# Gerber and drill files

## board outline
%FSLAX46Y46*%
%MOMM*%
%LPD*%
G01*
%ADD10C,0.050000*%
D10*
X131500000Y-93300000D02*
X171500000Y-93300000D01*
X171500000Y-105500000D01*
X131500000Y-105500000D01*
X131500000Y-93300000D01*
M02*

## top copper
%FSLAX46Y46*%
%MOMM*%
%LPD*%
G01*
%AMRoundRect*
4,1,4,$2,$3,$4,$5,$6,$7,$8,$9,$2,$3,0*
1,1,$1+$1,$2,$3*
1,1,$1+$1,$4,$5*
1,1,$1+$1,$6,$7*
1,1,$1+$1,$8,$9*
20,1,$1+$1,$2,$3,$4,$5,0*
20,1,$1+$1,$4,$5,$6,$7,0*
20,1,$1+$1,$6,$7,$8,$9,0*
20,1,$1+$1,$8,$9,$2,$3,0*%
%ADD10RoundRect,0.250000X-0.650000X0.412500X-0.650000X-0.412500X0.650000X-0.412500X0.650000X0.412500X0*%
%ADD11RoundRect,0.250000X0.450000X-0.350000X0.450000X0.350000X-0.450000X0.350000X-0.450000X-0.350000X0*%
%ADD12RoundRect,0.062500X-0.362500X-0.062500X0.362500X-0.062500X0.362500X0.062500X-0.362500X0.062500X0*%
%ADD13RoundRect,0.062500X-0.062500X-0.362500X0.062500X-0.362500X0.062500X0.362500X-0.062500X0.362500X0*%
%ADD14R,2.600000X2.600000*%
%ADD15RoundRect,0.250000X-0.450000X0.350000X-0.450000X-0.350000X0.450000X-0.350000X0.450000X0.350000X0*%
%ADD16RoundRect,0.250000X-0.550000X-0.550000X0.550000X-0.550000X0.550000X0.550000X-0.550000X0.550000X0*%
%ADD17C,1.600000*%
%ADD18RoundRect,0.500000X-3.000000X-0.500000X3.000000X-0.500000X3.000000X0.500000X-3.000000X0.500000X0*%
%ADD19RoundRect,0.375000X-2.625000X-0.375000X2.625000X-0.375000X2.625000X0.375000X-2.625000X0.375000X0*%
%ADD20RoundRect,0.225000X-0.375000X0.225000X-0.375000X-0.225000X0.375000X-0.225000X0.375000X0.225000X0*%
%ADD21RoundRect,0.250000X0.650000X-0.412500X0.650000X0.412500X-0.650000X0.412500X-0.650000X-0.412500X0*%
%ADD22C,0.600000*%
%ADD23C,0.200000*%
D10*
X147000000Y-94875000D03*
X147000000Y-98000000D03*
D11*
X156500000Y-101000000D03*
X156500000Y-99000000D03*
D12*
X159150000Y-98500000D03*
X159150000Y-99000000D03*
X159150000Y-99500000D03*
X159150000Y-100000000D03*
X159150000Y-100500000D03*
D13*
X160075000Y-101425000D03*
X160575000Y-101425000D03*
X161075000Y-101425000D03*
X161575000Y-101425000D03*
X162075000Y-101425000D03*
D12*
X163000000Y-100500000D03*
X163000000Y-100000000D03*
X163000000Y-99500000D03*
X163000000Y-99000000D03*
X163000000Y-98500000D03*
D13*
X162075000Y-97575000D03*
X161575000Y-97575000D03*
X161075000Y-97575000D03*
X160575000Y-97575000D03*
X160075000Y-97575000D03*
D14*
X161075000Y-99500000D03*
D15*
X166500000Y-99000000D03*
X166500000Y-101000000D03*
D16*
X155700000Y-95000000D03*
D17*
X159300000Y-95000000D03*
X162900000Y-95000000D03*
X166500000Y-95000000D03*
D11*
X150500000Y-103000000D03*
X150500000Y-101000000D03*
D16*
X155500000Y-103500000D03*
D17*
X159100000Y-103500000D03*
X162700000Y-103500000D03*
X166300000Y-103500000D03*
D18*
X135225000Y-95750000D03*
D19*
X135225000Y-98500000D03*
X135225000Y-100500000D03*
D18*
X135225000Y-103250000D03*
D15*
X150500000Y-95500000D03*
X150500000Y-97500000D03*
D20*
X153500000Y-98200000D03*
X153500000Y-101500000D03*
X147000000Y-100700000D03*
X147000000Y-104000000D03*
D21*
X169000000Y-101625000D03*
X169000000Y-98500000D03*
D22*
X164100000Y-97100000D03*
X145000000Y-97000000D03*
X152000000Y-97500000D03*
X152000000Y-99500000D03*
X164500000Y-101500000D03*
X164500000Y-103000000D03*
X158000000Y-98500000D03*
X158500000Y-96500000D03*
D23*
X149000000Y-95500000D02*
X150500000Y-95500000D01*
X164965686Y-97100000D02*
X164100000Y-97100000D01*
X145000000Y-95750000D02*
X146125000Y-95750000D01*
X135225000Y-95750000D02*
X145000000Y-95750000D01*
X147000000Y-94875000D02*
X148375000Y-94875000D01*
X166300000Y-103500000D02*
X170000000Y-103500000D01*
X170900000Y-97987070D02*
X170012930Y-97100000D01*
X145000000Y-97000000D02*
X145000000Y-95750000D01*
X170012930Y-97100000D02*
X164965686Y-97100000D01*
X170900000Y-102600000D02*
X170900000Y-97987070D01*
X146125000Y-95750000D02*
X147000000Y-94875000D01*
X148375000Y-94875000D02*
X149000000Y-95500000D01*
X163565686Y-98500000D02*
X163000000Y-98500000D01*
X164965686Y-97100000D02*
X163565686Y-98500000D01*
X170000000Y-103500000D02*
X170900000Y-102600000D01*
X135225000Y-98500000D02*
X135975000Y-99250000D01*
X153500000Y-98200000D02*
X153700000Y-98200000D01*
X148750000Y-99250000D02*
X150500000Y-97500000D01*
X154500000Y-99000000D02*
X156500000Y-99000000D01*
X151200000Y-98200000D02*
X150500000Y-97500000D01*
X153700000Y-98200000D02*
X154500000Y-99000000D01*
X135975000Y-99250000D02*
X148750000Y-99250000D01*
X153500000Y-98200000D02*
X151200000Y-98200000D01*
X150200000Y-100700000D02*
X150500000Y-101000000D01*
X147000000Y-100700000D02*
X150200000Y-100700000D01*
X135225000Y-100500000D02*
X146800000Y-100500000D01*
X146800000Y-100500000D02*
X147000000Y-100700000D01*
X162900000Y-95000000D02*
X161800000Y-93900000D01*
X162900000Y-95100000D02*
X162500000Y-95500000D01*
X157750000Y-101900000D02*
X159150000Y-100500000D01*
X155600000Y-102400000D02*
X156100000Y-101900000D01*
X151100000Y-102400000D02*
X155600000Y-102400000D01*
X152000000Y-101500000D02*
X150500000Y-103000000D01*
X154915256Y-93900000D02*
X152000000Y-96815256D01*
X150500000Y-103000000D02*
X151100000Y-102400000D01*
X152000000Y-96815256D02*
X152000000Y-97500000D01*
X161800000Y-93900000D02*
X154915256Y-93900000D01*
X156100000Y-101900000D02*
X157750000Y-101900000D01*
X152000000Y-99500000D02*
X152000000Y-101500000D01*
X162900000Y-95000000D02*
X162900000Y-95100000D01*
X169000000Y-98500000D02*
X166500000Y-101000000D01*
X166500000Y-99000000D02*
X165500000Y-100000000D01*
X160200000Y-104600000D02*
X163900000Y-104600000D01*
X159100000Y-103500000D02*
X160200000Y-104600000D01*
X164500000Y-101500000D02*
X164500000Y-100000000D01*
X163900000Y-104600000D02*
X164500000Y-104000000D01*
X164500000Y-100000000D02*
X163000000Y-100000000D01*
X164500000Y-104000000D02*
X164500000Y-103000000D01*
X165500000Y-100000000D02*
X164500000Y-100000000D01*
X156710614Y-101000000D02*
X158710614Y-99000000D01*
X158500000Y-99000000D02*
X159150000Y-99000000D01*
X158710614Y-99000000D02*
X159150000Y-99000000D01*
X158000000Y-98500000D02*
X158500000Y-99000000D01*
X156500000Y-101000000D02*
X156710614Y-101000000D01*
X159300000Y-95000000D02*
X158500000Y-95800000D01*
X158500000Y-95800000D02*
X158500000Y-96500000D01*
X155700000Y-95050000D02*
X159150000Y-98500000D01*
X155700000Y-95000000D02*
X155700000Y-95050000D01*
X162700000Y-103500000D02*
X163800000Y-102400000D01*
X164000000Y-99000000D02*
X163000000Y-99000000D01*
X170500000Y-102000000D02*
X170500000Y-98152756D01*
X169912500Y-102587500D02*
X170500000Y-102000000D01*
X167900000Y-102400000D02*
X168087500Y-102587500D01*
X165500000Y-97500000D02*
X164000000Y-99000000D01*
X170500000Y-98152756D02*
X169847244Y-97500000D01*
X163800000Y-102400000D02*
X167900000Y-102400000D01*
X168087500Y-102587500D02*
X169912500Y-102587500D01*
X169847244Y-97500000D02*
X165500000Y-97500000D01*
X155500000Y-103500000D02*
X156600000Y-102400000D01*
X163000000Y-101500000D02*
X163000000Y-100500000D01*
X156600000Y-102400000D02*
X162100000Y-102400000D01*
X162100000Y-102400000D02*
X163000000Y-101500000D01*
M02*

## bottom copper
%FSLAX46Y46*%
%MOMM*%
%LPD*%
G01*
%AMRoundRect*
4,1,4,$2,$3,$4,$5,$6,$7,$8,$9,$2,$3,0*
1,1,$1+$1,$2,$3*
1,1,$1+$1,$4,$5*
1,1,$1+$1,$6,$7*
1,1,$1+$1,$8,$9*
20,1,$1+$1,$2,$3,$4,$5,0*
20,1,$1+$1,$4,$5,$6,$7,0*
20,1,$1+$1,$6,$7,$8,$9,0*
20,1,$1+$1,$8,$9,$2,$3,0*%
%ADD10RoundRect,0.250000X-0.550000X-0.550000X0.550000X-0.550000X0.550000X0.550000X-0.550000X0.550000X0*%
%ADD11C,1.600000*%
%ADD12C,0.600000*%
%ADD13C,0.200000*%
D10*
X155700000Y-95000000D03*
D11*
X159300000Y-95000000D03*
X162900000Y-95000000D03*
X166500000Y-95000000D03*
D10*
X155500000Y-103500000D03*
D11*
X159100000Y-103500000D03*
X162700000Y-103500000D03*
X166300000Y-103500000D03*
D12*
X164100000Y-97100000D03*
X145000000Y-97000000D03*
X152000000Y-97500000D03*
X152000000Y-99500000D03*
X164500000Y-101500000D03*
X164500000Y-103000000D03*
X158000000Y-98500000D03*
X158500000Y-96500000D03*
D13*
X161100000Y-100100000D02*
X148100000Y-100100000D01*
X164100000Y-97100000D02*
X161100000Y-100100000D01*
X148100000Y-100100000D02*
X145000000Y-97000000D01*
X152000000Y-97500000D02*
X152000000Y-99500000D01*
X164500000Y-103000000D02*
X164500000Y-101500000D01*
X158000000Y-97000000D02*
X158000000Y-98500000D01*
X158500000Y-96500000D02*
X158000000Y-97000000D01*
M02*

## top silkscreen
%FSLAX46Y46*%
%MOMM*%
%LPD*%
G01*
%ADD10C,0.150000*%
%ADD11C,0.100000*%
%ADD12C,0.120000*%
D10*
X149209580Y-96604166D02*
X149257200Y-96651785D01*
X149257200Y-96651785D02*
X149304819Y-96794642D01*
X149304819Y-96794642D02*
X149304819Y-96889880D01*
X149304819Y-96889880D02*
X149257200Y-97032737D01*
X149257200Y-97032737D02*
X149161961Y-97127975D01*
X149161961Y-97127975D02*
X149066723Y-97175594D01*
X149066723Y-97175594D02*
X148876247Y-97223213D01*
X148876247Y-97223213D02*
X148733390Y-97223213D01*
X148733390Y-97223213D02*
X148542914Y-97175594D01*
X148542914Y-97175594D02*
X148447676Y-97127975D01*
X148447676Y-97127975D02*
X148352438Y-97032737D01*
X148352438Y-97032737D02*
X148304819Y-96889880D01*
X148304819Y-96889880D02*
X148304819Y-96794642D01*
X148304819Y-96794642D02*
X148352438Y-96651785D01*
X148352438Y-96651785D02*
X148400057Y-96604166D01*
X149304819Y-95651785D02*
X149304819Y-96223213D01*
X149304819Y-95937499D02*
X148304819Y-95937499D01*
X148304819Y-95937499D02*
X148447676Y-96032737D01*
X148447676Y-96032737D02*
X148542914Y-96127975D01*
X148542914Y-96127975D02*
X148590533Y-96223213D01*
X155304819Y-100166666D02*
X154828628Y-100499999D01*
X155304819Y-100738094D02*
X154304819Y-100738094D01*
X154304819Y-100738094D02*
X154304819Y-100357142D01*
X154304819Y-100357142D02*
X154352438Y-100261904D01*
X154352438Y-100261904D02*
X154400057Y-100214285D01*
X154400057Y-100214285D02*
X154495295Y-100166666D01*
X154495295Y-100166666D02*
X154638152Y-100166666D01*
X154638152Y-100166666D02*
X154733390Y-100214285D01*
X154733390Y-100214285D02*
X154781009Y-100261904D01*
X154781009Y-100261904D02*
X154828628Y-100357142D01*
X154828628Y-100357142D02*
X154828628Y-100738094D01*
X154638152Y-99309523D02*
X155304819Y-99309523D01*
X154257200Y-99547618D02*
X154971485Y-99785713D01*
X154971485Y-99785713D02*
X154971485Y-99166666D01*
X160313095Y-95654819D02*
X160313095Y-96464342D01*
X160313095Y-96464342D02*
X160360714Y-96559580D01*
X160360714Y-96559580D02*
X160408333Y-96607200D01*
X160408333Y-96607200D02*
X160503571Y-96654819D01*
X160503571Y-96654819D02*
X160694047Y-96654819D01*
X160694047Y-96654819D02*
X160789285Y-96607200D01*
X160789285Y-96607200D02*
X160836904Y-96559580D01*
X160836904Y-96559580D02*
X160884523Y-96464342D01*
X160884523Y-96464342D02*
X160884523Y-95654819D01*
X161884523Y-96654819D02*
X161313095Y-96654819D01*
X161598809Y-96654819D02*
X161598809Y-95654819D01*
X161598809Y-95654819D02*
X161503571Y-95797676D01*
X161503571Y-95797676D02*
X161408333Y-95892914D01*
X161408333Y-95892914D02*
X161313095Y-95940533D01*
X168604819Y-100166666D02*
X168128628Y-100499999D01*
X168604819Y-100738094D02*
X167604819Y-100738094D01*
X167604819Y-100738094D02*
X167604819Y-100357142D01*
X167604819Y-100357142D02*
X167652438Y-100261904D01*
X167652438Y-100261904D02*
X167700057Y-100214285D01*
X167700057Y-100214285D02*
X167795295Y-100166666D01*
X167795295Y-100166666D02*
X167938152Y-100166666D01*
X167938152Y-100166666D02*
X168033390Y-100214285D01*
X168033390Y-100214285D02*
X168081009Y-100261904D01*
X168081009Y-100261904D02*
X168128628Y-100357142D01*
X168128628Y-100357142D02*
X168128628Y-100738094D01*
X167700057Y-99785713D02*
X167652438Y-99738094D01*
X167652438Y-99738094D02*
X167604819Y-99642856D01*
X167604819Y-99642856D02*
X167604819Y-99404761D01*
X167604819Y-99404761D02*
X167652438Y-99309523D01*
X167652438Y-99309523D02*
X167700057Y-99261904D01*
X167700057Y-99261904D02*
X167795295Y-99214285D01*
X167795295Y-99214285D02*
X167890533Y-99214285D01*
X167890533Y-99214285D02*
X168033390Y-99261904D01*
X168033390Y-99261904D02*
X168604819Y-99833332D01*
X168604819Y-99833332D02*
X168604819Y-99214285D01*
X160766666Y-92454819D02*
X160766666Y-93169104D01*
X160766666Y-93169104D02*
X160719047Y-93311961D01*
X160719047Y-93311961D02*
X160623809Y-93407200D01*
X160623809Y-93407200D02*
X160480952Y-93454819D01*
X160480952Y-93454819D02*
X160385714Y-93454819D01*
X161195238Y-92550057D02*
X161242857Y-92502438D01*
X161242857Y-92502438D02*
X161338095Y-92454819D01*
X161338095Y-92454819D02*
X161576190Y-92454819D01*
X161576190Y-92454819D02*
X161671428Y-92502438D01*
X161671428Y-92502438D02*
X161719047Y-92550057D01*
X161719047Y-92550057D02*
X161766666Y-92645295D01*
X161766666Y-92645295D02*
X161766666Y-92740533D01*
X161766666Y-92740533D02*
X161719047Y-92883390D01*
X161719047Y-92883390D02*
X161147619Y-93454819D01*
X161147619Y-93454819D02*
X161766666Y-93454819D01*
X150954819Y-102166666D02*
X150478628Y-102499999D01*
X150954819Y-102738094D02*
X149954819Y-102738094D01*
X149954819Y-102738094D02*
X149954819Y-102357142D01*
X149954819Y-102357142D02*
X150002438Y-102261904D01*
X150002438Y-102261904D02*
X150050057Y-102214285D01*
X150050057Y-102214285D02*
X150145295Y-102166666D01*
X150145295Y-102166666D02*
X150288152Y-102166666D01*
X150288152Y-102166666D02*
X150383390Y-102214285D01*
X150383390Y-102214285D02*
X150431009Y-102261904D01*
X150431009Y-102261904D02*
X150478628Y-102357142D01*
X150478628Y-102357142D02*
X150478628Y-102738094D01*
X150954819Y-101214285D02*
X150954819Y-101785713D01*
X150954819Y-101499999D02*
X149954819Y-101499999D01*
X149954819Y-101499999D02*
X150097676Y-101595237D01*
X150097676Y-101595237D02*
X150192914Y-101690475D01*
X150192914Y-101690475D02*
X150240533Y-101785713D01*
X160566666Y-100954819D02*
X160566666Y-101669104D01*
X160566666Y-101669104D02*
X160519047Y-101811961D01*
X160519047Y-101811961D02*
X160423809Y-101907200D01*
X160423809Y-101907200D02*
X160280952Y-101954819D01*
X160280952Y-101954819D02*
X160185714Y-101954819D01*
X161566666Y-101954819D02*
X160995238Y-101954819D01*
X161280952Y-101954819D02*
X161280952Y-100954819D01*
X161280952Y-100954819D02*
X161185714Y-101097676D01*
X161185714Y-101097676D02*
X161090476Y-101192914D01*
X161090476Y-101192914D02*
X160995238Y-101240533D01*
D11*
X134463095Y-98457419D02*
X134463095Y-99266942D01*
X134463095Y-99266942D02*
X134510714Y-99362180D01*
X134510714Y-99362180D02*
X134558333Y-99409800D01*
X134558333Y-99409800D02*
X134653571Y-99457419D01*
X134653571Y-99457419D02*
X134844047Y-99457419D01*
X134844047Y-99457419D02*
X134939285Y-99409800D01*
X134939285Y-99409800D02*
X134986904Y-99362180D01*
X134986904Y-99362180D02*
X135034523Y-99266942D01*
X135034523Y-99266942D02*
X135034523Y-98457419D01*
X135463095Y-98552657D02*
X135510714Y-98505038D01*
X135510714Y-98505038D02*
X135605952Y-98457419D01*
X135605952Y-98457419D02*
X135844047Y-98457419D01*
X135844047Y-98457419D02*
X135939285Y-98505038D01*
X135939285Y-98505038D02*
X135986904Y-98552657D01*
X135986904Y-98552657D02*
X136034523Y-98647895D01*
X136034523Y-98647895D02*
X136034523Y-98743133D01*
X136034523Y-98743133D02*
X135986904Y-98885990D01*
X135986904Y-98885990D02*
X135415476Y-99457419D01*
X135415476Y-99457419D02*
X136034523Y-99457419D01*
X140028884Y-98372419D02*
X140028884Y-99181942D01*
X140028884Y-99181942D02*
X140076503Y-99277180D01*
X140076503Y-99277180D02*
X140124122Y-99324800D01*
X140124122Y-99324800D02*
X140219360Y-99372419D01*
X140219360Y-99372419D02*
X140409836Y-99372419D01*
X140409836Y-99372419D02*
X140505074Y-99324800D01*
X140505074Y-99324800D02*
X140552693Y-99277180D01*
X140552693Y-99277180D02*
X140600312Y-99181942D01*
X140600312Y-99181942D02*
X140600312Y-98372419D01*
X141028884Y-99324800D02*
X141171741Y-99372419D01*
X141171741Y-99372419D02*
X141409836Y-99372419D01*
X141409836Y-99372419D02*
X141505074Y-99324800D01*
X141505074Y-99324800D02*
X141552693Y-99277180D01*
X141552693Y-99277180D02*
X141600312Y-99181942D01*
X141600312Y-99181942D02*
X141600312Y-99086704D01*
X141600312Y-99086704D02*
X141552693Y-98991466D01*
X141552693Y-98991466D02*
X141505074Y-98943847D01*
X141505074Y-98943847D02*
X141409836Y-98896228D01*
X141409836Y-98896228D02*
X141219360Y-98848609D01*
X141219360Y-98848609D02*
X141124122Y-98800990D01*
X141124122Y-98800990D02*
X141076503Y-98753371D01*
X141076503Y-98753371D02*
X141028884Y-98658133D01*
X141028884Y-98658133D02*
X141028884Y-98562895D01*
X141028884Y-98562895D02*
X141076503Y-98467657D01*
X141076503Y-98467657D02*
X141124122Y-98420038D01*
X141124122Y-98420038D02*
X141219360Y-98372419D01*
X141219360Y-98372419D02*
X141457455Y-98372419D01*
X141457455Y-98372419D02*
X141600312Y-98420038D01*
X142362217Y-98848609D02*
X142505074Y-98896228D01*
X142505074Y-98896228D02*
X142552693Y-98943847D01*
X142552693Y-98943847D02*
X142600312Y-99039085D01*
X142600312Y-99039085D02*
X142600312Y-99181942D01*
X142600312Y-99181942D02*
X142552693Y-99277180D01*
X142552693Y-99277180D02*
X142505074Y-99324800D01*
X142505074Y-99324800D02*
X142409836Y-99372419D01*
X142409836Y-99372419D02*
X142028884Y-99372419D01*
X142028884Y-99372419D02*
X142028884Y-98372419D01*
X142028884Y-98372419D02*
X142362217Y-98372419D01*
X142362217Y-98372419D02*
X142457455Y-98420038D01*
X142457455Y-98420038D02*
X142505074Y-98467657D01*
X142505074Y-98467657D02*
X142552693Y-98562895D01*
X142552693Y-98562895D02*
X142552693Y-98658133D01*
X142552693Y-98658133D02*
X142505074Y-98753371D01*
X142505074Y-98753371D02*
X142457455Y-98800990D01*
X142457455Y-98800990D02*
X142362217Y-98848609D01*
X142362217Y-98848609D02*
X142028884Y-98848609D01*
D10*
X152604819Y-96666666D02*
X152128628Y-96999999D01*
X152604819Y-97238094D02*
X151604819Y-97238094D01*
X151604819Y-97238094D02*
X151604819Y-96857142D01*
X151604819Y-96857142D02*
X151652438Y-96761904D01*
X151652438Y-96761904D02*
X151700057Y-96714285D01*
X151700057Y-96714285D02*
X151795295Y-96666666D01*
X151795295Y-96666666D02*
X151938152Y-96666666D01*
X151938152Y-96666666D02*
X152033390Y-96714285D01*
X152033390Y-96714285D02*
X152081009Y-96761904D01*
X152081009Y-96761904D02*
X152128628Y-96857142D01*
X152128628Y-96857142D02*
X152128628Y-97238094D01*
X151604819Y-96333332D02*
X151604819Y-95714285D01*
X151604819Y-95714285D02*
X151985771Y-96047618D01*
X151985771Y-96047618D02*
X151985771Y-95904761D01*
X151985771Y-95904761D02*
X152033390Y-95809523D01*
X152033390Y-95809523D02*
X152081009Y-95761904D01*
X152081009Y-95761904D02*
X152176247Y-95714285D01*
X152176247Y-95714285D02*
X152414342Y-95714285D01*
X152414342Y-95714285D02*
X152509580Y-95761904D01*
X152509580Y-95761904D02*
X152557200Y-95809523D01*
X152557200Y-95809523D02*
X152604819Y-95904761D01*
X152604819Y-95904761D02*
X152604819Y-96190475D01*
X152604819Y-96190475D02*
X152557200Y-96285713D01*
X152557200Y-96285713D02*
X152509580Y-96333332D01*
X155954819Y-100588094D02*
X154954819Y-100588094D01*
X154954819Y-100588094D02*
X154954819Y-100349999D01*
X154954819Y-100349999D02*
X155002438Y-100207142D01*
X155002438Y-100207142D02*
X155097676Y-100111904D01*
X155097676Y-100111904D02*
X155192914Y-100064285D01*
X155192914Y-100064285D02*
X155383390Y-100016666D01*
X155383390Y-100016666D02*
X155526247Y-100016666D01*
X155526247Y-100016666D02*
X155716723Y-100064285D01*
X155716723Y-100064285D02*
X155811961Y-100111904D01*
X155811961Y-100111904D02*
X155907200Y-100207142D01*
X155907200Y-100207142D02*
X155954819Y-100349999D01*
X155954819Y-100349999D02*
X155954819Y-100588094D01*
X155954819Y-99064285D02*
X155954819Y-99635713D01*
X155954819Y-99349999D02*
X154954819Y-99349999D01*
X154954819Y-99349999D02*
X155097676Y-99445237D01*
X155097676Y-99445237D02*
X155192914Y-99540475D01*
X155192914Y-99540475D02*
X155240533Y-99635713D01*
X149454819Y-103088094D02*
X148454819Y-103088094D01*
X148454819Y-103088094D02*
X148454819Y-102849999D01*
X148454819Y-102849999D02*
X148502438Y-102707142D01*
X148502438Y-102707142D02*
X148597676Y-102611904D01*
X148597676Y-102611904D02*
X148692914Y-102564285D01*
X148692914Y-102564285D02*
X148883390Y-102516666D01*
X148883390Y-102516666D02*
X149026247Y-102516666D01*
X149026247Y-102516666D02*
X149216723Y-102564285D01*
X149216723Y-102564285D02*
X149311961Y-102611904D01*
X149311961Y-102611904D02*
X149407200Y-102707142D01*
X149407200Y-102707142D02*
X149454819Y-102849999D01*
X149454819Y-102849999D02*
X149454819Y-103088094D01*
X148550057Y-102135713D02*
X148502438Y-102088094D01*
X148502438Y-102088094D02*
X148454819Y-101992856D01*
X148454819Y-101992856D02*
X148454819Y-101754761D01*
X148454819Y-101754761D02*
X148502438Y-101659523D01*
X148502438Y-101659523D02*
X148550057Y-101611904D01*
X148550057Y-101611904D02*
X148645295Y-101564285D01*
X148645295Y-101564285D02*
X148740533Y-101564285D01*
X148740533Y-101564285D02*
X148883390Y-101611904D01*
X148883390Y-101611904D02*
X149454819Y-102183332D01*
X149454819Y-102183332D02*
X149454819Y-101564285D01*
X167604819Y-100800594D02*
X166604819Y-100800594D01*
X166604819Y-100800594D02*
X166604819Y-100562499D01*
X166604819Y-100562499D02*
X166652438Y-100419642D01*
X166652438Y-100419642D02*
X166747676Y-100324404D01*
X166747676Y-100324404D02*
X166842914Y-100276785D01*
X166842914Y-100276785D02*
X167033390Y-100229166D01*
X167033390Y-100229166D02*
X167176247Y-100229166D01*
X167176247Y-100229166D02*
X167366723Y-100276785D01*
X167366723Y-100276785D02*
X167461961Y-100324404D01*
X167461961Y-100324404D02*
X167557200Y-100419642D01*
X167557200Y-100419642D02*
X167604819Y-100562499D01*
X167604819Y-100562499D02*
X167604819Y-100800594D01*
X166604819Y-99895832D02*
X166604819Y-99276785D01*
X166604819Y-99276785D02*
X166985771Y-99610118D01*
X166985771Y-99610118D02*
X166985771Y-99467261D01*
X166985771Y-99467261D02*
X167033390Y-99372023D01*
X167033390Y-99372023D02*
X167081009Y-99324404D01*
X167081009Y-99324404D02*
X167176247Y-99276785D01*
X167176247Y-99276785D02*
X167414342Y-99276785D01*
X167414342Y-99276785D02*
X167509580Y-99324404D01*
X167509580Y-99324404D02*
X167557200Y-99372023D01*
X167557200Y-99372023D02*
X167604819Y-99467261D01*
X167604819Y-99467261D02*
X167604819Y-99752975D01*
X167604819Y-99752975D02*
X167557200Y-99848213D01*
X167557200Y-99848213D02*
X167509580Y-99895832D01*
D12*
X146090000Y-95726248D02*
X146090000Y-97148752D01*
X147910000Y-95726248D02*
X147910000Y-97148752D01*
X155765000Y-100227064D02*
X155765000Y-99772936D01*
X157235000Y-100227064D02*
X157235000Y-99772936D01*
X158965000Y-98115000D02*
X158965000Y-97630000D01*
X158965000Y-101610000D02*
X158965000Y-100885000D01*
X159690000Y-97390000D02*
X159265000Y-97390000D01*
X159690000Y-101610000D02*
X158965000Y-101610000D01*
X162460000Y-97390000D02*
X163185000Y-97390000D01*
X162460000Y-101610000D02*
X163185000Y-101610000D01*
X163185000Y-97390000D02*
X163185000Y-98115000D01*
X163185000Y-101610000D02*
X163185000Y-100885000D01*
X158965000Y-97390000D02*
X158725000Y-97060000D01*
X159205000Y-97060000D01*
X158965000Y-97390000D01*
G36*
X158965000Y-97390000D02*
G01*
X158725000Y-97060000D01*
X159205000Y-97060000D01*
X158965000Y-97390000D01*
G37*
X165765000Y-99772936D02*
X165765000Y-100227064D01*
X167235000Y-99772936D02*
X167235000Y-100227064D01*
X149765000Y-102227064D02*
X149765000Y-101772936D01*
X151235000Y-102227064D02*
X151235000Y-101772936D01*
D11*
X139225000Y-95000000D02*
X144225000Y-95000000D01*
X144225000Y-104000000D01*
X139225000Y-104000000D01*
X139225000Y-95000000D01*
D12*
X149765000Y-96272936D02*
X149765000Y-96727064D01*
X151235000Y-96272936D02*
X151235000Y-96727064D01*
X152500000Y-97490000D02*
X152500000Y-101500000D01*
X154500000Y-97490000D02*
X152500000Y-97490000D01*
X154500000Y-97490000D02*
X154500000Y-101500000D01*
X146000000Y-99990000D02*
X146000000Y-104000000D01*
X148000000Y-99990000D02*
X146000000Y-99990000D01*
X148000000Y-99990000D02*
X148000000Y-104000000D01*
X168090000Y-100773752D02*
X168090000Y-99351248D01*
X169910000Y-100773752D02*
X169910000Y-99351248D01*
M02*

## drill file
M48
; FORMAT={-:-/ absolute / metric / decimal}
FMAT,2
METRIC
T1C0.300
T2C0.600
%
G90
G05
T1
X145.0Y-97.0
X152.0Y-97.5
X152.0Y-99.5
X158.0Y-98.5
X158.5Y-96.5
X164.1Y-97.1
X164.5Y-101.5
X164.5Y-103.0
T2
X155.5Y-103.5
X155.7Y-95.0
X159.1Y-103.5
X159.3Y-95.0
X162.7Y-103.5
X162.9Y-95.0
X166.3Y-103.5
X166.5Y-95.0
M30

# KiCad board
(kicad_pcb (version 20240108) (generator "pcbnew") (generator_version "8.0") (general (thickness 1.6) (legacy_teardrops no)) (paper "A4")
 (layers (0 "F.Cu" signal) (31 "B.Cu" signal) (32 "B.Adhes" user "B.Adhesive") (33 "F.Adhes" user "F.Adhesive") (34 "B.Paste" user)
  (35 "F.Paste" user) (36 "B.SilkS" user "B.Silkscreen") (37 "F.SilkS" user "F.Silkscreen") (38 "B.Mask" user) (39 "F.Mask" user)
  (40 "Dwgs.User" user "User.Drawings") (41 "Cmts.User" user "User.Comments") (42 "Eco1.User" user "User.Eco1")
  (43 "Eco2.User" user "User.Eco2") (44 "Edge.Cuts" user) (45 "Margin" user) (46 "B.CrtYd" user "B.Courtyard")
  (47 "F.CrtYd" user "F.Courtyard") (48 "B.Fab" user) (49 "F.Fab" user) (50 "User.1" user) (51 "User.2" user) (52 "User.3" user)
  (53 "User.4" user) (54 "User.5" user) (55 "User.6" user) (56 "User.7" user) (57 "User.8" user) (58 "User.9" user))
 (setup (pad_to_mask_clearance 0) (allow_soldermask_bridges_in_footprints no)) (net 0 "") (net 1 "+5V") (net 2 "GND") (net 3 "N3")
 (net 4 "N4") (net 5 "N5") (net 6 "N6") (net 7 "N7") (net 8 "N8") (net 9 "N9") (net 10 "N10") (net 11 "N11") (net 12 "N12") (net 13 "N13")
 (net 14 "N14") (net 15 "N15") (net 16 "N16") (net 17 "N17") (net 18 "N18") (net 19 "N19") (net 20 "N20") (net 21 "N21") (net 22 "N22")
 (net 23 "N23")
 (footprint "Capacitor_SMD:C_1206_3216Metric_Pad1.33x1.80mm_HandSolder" (layer "F.Cu") (at 147 96.4375 -90)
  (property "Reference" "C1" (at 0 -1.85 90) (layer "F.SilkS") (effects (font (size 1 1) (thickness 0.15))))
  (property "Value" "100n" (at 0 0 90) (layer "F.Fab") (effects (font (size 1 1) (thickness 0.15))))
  (fp_line (start -0.711252 0.91) (end 0.711252 0.91) (stroke (width 0.12) (type solid)) (layer "F.SilkS"))
  (fp_line (start -0.711252 -0.91) (end 0.711252 -0.91) (stroke (width 0.12) (type solid)) (layer "F.SilkS"))
  (pad "1" smd roundrect (at -1.5625 0 270) (size 1.325 1.8) (layers "F.Cu" "F.Paste" "F.Mask") (roundrect_rratio 0.188679) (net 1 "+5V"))
  (pad "2" smd roundrect (at 1.5625 0 270) (size 1.325 1.8) (layers "F.Cu" "F.Paste" "F.Mask") (roundrect_rratio 0.188679) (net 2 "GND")))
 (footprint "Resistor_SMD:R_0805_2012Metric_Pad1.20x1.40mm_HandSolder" (layer "F.Cu") (at 156.5 100 90)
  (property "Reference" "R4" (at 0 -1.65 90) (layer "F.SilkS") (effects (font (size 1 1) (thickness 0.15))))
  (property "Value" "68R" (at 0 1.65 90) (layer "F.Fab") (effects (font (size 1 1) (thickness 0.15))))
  (fp_line (start -0.227064 -0.735) (end 0.227064 -0.735) (stroke (width 0.12) (type solid)) (layer "F.SilkS"))
  (fp_line (start -0.227064 0.735) (end 0.227064 0.735) (stroke (width 0.12) (type solid)) (layer "F.SilkS"))
  (pad "1" smd roundrect (at -1 0 90) (size 1.2 1.4) (layers "F.Cu" "F.Paste" "F.Mask") (roundrect_rratio 0.208333) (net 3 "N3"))
  (pad "2" smd roundrect (at 1 0 90) (size 1.2 1.4) (layers "F.Cu" "F.Paste" "F.Mask") (roundrect_rratio 0.208333) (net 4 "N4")))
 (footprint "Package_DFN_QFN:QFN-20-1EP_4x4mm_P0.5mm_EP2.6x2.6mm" (layer "F.Cu") (at 161.075 99.5)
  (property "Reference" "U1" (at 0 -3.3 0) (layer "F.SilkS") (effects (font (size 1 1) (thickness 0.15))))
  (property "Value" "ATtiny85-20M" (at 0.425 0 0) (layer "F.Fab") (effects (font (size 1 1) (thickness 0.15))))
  (fp_line (start -2.11 -1.385) (end -2.11 -1.87) (stroke (width 0.12) (type solid)) (layer "F.SilkS"))
  (fp_line (start -2.11 2.11) (end -2.11 1.385) (stroke (width 0.12) (type solid)) (layer "F.SilkS"))
  (fp_line (start -1.385 -2.11) (end -1.81 -2.11) (stroke (width 0.12) (type solid)) (layer "F.SilkS"))
  (fp_line (start -1.385 2.11) (end -2.11 2.11) (stroke (width 0.12) (type solid)) (layer "F.SilkS"))
  (fp_line (start 1.385 -2.11) (end 2.11 -2.11) (stroke (width 0.12) (type solid)) (layer "F.SilkS"))
  (fp_line (start 1.385 2.11) (end 2.11 2.11) (stroke (width 0.12) (type solid)) (layer "F.SilkS"))
  (fp_line (start 2.11 -2.11) (end 2.11 -1.385) (stroke (width 0.12) (type solid)) (layer "F.SilkS"))
  (fp_line (start 2.11 2.11) (end 2.11 1.385) (stroke (width 0.12) (type solid)) (layer "F.SilkS"))
  (fp_poly
   (pts (xy -2.11 -2.11) (xy -2.35 -2.44) (xy -1.87 -2.44) (xy -2.11 -2.11)) (stroke (width 0.12) (type solid)) (fill solid)
   (layer "F.SilkS"))
  (pad "" smd roundrect (at -0.65 -0.65) (size 1.05 1.05) (layers "F.Paste") (roundrect_rratio 0.238095))
  (pad "" smd roundrect (at -0.65 0.65) (size 1.05 1.05) (layers "F.Paste") (roundrect_rratio 0.238095))
  (pad "" smd roundrect (at 0.65 -0.65) (size 1.05 1.05) (layers "F.Paste") (roundrect_rratio 0.238095))
  (pad "" smd roundrect (at 0.65 0.65) (size 1.05 1.05) (layers "F.Paste") (roundrect_rratio 0.238095))
  (pad "1" smd roundrect (at -1.925 -1) (size 0.85 0.25) (layers "F.Cu" "F.Paste" "F.Mask") (roundrect_rratio 0.25) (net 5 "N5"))
  (pad "2" smd roundrect (at -1.925 -0.5) (size 0.85 0.25) (layers "F.Cu" "F.Paste" "F.Mask") (roundrect_rratio 0.25) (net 3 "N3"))
  (pad "3" smd roundrect (at -1.925 0) (size 0.85 0.25) (layers "F.Cu" "F.Paste" "F.Mask") (roundrect_rratio 0.25) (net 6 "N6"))
  (pad "4" smd roundrect (at -1.925 0.5) (size 0.85 0.25) (layers "F.Cu" "F.Paste" "F.Mask") (roundrect_rratio 0.25) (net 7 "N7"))
  (pad "5" smd roundrect (at -1.925 1) (size 0.85 0.25) (layers "F.Cu" "F.Paste" "F.Mask") (roundrect_rratio 0.25) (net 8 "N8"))
  (pad "6" smd roundrect (at -1 1.925) (size 0.25 0.85) (layers "F.Cu" "F.Paste" "F.Mask") (roundrect_rratio 0.25) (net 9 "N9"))
  (pad "7" smd roundrect (at -0.5 1.925) (size 0.25 0.85) (layers "F.Cu" "F.Paste" "F.Mask") (roundrect_rratio 0.25) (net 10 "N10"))
  (pad "8" smd roundrect (at 0 1.925) (size 0.25 0.85) (layers "F.Cu" "F.Paste" "F.Mask") (roundrect_rratio 0.25) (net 2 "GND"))
  (pad "9" smd roundrect (at 0.5 1.925) (size 0.25 0.85) (layers "F.Cu" "F.Paste" "F.Mask") (roundrect_rratio 0.25) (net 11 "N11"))
  (pad "10" smd roundrect (at 1 1.925) (size 0.25 0.85) (layers "F.Cu" "F.Paste" "F.Mask") (roundrect_rratio 0.25) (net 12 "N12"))
  (pad "11" smd roundrect (at 1.925 1) (size 0.85 0.25) (layers "F.Cu" "F.Paste" "F.Mask") (roundrect_rratio 0.25) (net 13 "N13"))
  (pad "12" smd roundrect (at 1.925 0.5) (size 0.85 0.25) (layers "F.Cu" "F.Paste" "F.Mask") (roundrect_rratio 0.25) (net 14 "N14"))
  (pad "13" smd roundrect (at 1.925 0) (size 0.85 0.25) (layers "F.Cu" "F.Paste" "F.Mask") (roundrect_rratio 0.25) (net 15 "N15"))
  (pad "14" smd roundrect (at 1.925 -0.5) (size 0.85 0.25) (layers "F.Cu" "F.Paste" "F.Mask") (roundrect_rratio 0.25) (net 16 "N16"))
  (pad "15" smd roundrect (at 1.925 -1) (size 0.85 0.25) (layers "F.Cu" "F.Paste" "F.Mask") (roundrect_rratio 0.25) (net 1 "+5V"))
  (pad "16" smd roundrect (at 1 -1.925) (size 0.25 0.85) (layers "F.Cu" "F.Paste" "F.Mask") (roundrect_rratio 0.25) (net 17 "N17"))
  (pad "17" smd roundrect (at 0.5 -1.925) (size 0.25 0.85) (layers "F.Cu" "F.Paste" "F.Mask") (roundrect_rratio 0.25) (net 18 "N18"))
  (pad "18" smd roundrect (at 0 -1.925) (size 0.25 0.85) (layers "F.Cu" "F.Paste" "F.Mask") (roundrect_rratio 0.25) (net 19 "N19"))
  (pad "19" smd roundrect (at -0.5 -1.925) (size 0.25 0.85) (layers "F.Cu" "F.Paste" "F.Mask") (roundrect_rratio 0.25) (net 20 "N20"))
  (pad "20" smd roundrect (at -1 -1.925) (size 0.25 0.85) (layers "F.Cu" "F.Paste" "F.Mask") (roundrect_rratio 0.25) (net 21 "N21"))
  (pad "21" smd rect (at 0 0) (size 2.6 2.6) (layers "F.Cu" "F.Mask") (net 2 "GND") (zone_connect 2)))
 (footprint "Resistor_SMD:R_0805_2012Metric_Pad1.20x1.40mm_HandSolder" (layer "F.Cu") (at 166.5 100 -90)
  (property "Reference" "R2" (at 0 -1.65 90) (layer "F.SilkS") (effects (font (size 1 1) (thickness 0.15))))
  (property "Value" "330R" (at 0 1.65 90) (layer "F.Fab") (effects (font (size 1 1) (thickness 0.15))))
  (fp_line (start -0.227064 0.735) (end 0.227064 0.735) (stroke (width 0.12) (type solid)) (layer "F.SilkS"))
  (fp_line (start -0.227064 -0.735) (end 0.227064 -0.735) (stroke (width 0.12) (type solid)) (layer "F.SilkS"))
  (pad "1" smd roundrect (at -1 0 270) (size 1.2 1.4) (layers "F.Cu" "F.Paste" "F.Mask") (roundrect_rratio 0.208333) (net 14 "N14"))
  (pad "2" smd roundrect (at 1 0 270) (size 1.2 1.4) (layers "F.Cu" "F.Paste" "F.Mask") (roundrect_rratio 0.208333) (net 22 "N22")))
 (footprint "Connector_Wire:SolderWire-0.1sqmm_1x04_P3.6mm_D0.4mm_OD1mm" (layer "F.Cu") (at 155.7 95)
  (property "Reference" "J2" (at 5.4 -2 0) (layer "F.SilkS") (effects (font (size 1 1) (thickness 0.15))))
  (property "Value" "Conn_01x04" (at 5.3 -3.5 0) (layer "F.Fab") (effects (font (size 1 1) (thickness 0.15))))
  (pad "1" thru_hole roundrect (at 0 0) (size 1.6 1.6) (drill 0.6) (layers "*.Cu" "*.Mask") (remove_unused_layers no)
   (roundrect_rratio 0.15625) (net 5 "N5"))
  (pad "2" thru_hole circle (at 3.6 0) (size 1.6 1.6) (drill 0.6) (layers "*.Cu" "*.Mask") (remove_unused_layers no) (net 3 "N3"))
  (pad "3" thru_hole circle (at 7.2 0) (size 1.6 1.6) (drill 0.6) (layers "*.Cu" "*.Mask") (remove_unused_layers no) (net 8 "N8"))
  (pad "4" thru_hole circle (at 10.8 0) (size 1.6 1.6) (drill 0.6) (layers "*.Cu" "*.Mask") (remove_unused_layers no) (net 2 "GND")))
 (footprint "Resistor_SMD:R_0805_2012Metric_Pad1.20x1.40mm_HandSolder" (layer "F.Cu") (at 150.5 102 90)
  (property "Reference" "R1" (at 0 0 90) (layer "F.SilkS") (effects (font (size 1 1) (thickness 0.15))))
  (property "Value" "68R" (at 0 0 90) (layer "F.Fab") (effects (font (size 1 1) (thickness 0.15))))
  (fp_line (start -0.227064 -0.735) (end 0.227064 -0.735) (stroke (width 0.12) (type solid)) (layer "F.SilkS"))
  (fp_line (start -0.227064 0.735) (end 0.227064 0.735) (stroke (width 0.12) (type solid)) (layer "F.SilkS"))
  (pad "1" smd roundrect (at -1 0 90) (size 1.2 1.4) (layers "F.Cu" "F.Paste" "F.Mask") (roundrect_rratio 0.208333) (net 8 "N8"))
  (pad "2" smd roundrect (at 1 0 90) (size 1.2 1.4) (layers "F.Cu" "F.Paste" "F.Mask") (roundrect_rratio 0.208333) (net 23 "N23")))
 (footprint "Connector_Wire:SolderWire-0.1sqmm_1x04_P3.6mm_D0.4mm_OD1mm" (layer "F.Cu") (at 155.5 103.5)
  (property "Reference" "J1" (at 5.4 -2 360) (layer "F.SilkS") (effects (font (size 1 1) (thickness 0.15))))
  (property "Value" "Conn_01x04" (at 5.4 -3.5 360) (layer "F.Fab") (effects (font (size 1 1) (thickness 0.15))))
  (pad "1" thru_hole roundrect (at 0 0) (size 1.6 1.6) (drill 0.6) (layers "*.Cu" "*.Mask") (remove_unused_layers no)
   (roundrect_rratio 0.15625) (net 13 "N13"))
  (pad "2" thru_hole circle (at 3.6 0) (size 1.6 1.6) (drill 0.6) (layers "*.Cu" "*.Mask") (remove_unused_layers no) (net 14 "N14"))
  (pad "3" thru_hole circle (at 7.2 0) (size 1.6 1.6) (drill 0.6) (layers "*.Cu" "*.Mask") (remove_unused_layers no) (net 16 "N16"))
  (pad "4" thru_hole circle (at 10.8 0) (size 1.6 1.6) (drill 0.6) (layers "*.Cu" "*.Mask") (remove_unused_layers no) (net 1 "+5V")))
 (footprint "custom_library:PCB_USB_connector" (layer "F.Cu") (at 135.225 99.5)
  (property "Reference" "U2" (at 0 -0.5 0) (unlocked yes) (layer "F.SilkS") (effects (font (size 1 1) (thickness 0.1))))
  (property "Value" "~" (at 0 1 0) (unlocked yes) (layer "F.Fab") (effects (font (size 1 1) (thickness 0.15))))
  (fp_rect (start 4 -4.5) (end 9 4.5) (stroke (width 0.1) (type default)) (fill none) (layer "F.SilkS"))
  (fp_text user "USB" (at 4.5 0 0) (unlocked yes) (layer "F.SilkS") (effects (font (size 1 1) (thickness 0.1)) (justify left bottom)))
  (pad "1" smd roundrect (at 0 -3.75) (size 7 2) (layers "F.Cu" "F.Paste" "F.Mask") (roundrect_rratio 0.25) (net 1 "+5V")
   (thermal_bridge_angle 45))
  (pad "2" smd roundrect (at 0 -1) (size 6 1.5) (layers "F.Cu" "F.Paste" "F.Mask") (roundrect_rratio 0.25) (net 4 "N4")
   (thermal_bridge_angle 45))
  (pad "3" smd roundrect (at 0 1) (size 6 1.5) (layers "F.Cu" "F.Paste" "F.Mask") (roundrect_rratio 0.25) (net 23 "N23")
   (thermal_bridge_angle 45))
  (pad "4" smd roundrect (at 0 3.75) (size 7 2) (layers "F.Cu" "F.Paste" "F.Mask") (roundrect_rratio 0.25) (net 2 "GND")
   (thermal_bridge_angle 45)))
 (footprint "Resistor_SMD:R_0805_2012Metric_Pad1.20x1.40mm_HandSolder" (layer "F.Cu") (at 150.5 96.5 -90)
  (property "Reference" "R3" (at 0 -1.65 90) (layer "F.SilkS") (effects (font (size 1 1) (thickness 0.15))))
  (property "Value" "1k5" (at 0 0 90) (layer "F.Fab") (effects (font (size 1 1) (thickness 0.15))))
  (fp_line (start -0.227064 0.735) (end 0.227064 0.735) (stroke (width 0.12) (type solid)) (layer "F.SilkS"))
  (fp_line (start -0.227064 -0.735) (end 0.227064 -0.735) (stroke (width 0.12) (type solid)) (layer "F.SilkS"))
  (pad "1" smd roundrect (at -1 0 270) (size 1.2 1.4) (layers "F.Cu" "F.Paste" "F.Mask") (roundrect_rratio 0.208333) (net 1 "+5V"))
  (pad "2" smd roundrect (at 1 0 270) (size 1.2 1.4) (layers "F.Cu" "F.Paste" "F.Mask") (roundrect_rratio 0.208333) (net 4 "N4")))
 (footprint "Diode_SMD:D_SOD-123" (layer "F.Cu") (at 153.5 99.85 -90)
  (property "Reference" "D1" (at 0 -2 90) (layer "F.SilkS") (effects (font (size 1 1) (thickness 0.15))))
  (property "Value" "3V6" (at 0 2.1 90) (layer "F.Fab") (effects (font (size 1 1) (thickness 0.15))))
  (fp_line (start -2.36 1) (end 1.65 1) (stroke (width 0.12) (type solid)) (layer "F.SilkS"))
  (fp_line (start -2.36 -1) (end -2.36 1) (stroke (width 0.12) (type solid)) (layer "F.SilkS"))
  (fp_line (start -2.36 -1) (end 1.65 -1) (stroke (width 0.12) (type solid)) (layer "F.SilkS"))
  (pad "1" smd roundrect (at -1.65 0 270) (size 0.9 1.2) (layers "F.Cu" "F.Paste" "F.Mask") (roundrect_rratio 0.25) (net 4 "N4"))
  (pad "2" smd roundrect (at 1.65 0 270) (size 0.9 1.2) (layers "F.Cu" "F.Paste" "F.Mask") (roundrect_rratio 0.25) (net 2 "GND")))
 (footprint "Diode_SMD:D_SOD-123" (layer "F.Cu") (at 147 102.35 -90)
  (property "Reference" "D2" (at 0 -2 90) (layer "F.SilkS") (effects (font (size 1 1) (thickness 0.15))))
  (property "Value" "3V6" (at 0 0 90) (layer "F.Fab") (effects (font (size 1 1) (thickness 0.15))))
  (fp_line (start -2.36 1) (end 1.65 1) (stroke (width 0.12) (type solid)) (layer "F.SilkS"))
  (fp_line (start -2.36 -1) (end -2.36 1) (stroke (width 0.12) (type solid)) (layer "F.SilkS"))
  (fp_line (start -2.36 -1) (end 1.65 -1) (stroke (width 0.12) (type solid)) (layer "F.SilkS"))
  (pad "1" smd roundrect (at -1.65 0 270) (size 0.9 1.2) (layers "F.Cu" "F.Paste" "F.Mask") (roundrect_rratio 0.25) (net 23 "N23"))
  (pad "2" smd roundrect (at 1.65 0 270) (size 0.9 1.2) (layers "F.Cu" "F.Paste" "F.Mask") (roundrect_rratio 0.25) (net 2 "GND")))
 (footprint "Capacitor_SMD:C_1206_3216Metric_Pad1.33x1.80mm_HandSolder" (layer "F.Cu") (at 169 100.0625 90)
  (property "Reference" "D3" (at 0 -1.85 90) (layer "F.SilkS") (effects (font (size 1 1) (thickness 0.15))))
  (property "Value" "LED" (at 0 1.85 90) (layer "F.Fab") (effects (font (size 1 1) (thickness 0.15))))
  (fp_line (start -0.711252 -0.91) (end 0.711252 -0.91) (stroke (width 0.12) (type solid)) (layer "F.SilkS"))
  (fp_line (start -0.711252 0.91) (end 0.711252 0.91) (stroke (width 0.12) (type solid)) (layer "F.SilkS"))
  (pad "1" smd roundrect (at -1.5625 0 90) (size 1.325 1.8) (layers "F.Cu" "F.Paste" "F.Mask") (roundrect_rratio 0.188679) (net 2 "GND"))
  (pad "2" smd roundrect (at 1.5625 0 90) (size 1.325 1.8) (layers "F.Cu" "F.Paste" "F.Mask") (roundrect_rratio 0.188679) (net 22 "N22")))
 (gr_rect (start 131.5 93.3) (end 171.5 105.5) (stroke (width 0.05) (type default)) (fill none) (layer "Edge.Cuts"))
 (segment (start 149 95.5) (end 150.5 95.5) (width 0.2) (layer "F.Cu") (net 1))
 (segment (start 164.965686 97.1) (end 164.1 97.1) (width 0.2) (layer "F.Cu") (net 1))
 (segment (start 145 95.75) (end 146.125 95.75) (width 0.2) (layer "F.Cu") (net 1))
 (segment (start 135.225 95.75) (end 145 95.75) (width 0.2) (layer "F.Cu") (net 1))
 (segment (start 147 94.875) (end 148.375 94.875) (width 0.2) (layer "F.Cu") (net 1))
 (segment (start 166.3 103.5) (end 170 103.5) (width 0.2) (layer "F.Cu") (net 1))
 (segment (start 170.9 97.98707) (end 170.01293 97.1) (width 0.2) (layer "F.Cu") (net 1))
 (segment (start 145 97) (end 145 95.75) (width 0.2) (layer "F.Cu") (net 1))
 (segment (start 170.01293 97.1) (end 164.965686 97.1) (width 0.2) (layer "F.Cu") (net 1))
 (segment (start 170.9 102.6) (end 170.9 97.98707) (width 0.2) (layer "F.Cu") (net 1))
 (segment (start 146.125 95.75) (end 147 94.875) (width 0.2) (layer "F.Cu") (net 1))
 (segment (start 148.375 94.875) (end 149 95.5) (width 0.2) (layer "F.Cu") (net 1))
 (segment (start 163.565686 98.5) (end 163 98.5) (width 0.2) (layer "F.Cu") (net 1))
 (segment (start 164.965686 97.1) (end 163.565686 98.5) (width 0.2) (layer "F.Cu") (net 1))
 (segment (start 170 103.5) (end 170.9 102.6) (width 0.2) (layer "F.Cu") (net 1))
 (via (at 164.1 97.1) (size 0.6) (drill 0.3) (layers "F.Cu" "B.Cu") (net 1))
 (via (at 145 97) (size 0.6) (drill 0.3) (layers "F.Cu" "B.Cu") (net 1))
 (segment (start 161.1 100.1) (end 148.1 100.1) (width 0.2) (layer "B.Cu") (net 1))
 (segment (start 164.1 97.1) (end 161.1 100.1) (width 0.2) (layer "B.Cu") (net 1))
 (segment (start 148.1 100.1) (end 145 97) (width 0.2) (layer "B.Cu") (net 1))
 (segment (start 135.225 98.5) (end 135.975 99.25) (width 0.2) (layer "F.Cu") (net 4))
 (segment (start 153.5 98.2) (end 153.7 98.2) (width 0.2) (layer "F.Cu") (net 4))
 (segment (start 148.75 99.25) (end 150.5 97.5) (width 0.2) (layer "F.Cu") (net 4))
 (segment (start 154.5 99) (end 156.5 99) (width 0.2) (layer "F.Cu") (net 4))
 (segment (start 151.2 98.2) (end 150.5 97.5) (width 0.2) (layer "F.Cu") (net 4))
 (segment (start 153.7 98.2) (end 154.5 99) (width 0.2) (layer "F.Cu") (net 4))
 (segment (start 135.975 99.25) (end 148.75 99.25) (width 0.2) (layer "F.Cu") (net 4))
 (segment (start 153.5 98.2) (end 151.2 98.2) (width 0.2) (layer "F.Cu") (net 4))
 (segment (start 150.2 100.7) (end 150.5 101) (width 0.2) (layer "F.Cu") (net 23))
 (segment (start 147 100.7) (end 150.2 100.7) (width 0.2) (layer "F.Cu") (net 23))
 (segment (start 135.225 100.5) (end 146.8 100.5) (width 0.2) (layer "F.Cu") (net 23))
 (segment (start 146.8 100.5) (end 147 100.7) (width 0.2) (layer "F.Cu") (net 23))
 (segment (start 162.9 95) (end 161.8 93.9) (width 0.2) (layer "F.Cu") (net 8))
 (segment (start 162.9 95.1) (end 162.5 95.5) (width 0.2) (layer "F.Cu") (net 8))
 (segment (start 157.75 101.9) (end 159.15 100.5) (width 0.2) (layer "F.Cu") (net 8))
 (segment (start 155.6 102.4) (end 156.1 101.9) (width 0.2) (layer "F.Cu") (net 8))
 (segment (start 151.1 102.4) (end 155.6 102.4) (width 0.2) (layer "F.Cu") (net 8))
 (segment (start 152 101.5) (end 150.5 103) (width 0.2) (layer "F.Cu") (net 8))
 (segment (start 154.915256 93.9) (end 152 96.815256) (width 0.2) (layer "F.Cu") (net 8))
 (segment (start 150.5 103) (end 151.1 102.4) (width 0.2) (layer "F.Cu") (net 8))
 (segment (start 152 96.815256) (end 152 97.5) (width 0.2) (layer "F.Cu") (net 8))
 (segment (start 161.8 93.9) (end 154.915256 93.9) (width 0.2) (layer "F.Cu") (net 8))
 (segment (start 156.1 101.9) (end 157.75 101.9) (width 0.2) (layer "F.Cu") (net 8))
 (segment (start 152 99.5) (end 152 101.5) (width 0.2) (layer "F.Cu") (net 8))
 (segment (start 162.9 95) (end 162.9 95.1) (width 0.2) (layer "F.Cu") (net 8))
 (via (at 152 97.5) (size 0.6) (drill 0.3) (layers "F.Cu" "B.Cu") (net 8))
 (via (at 152 99.5) (size 0.6) (drill 0.3) (layers "F.Cu" "B.Cu") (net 8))
 (segment (start 152 97.5) (end 152 99.5) (width 0.2) (layer "B.Cu") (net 8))
 (segment (start 169 98.5) (end 166.5 101) (width 0.2) (layer "F.Cu") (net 22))
 (segment (start 166.5 99) (end 165.5 100) (width 0.2) (layer "F.Cu") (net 14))
 (segment (start 160.2 104.6) (end 163.9 104.6) (width 0.2) (layer "F.Cu") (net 14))
 (segment (start 159.1 103.5) (end 160.2 104.6) (width 0.2) (layer "F.Cu") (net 14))
 (segment (start 164.5 101.5) (end 164.5 100) (width 0.2) (layer "F.Cu") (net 14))
 (segment (start 163.9 104.6) (end 164.5 104) (width 0.2) (layer "F.Cu") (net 14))
 (segment (start 164.5 100) (end 163 100) (width 0.2) (layer "F.Cu") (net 14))
 (segment (start 164.5 104) (end 164.5 103) (width 0.2) (layer "F.Cu") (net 14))
 (segment (start 165.5 100) (end 164.5 100) (width 0.2) (layer "F.Cu") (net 14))
 (via (at 164.5 101.5) (size 0.6) (drill 0.3) (layers "F.Cu" "B.Cu") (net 14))
 (via (at 164.5 103) (size 0.6) (drill 0.3) (layers "F.Cu" "B.Cu") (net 14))
 (segment (start 164.5 103) (end 164.5 101.5) (width 0.2) (layer "B.Cu") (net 14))
 (segment (start 156.710614 101) (end 158.710614 99) (width 0.2) (layer "F.Cu") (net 3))
 (segment (start 158.5 99) (end 159.15 99) (width 0.2) (layer "F.Cu") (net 3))
 (segment (start 158.710614 99) (end 159.15 99) (width 0.2) (layer "F.Cu") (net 3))
 (segment (start 158 98.5) (end 158.5 99) (width 0.2) (layer "F.Cu") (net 3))
 (segment (start 156.5 101) (end 156.710614 101) (width 0.2) (layer "F.Cu") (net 3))
 (segment (start 159.3 95) (end 158.5 95.8) (width 0.2) (layer "F.Cu") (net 3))
 (segment (start 158.5 95.8) (end 158.5 96.5) (width 0.2) (layer "F.Cu") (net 3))
 (via (at 158 98.5) (size 0.6) (drill 0.3) (layers "F.Cu" "B.Cu") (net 3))
 (via (at 158.5 96.5) (size 0.6) (drill 0.3) (layers "F.Cu" "B.Cu") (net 3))
 (segment (start 158 97) (end 158 98.5) (width 0.2) (layer "B.Cu") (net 3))
 (segment (start 158.5 96.5) (end 158 97) (width 0.2) (layer "B.Cu") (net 3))
 (segment (start 155.7 95.05) (end 159.15 98.5) (width 0.2) (layer "F.Cu") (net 5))
 (segment (start 155.7 95) (end 155.7 95.05) (width 0.2) (layer "F.Cu") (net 5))
 (segment (start 162.7 103.5) (end 163.8 102.4) (width 0.2) (layer "F.Cu") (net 16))
 (segment (start 164 99) (end 163 99) (width 0.2) (layer "F.Cu") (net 16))
 (segment (start 170.5 102) (end 170.5 98.152756) (width 0.2) (layer "F.Cu") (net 16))
 (segment (start 169.9125 102.5875) (end 170.5 102) (width 0.2) (layer "F.Cu") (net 16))
 (segment (start 167.9 102.4) (end 168.0875 102.5875) (width 0.2) (layer "F.Cu") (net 16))
 (segment (start 165.5 97.5) (end 164 99) (width 0.2) (layer "F.Cu") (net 16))
 (segment (start 170.5 98.152756) (end 169.847244 97.5) (width 0.2) (layer "F.Cu") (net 16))
 (segment (start 163.8 102.4) (end 167.9 102.4) (width 0.2) (layer "F.Cu") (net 16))
 (segment (start 168.0875 102.5875) (end 169.9125 102.5875) (width 0.2) (layer "F.Cu") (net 16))
 (segment (start 169.847244 97.5) (end 165.5 97.5) (width 0.2) (layer "F.Cu") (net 16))
 (segment (start 155.5 103.5) (end 156.6 102.4) (width 0.2) (layer "F.Cu") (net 13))
 (segment (start 163 101.5) (end 163 100.5) (width 0.2) (layer "F.Cu") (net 13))
 (segment (start 156.6 102.4) (end 162.1 102.4) (width 0.2) (layer "F.Cu") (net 13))
 (segment (start 162.1 102.4) (end 163 101.5) (width 0.2) (layer "F.Cu") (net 13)))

